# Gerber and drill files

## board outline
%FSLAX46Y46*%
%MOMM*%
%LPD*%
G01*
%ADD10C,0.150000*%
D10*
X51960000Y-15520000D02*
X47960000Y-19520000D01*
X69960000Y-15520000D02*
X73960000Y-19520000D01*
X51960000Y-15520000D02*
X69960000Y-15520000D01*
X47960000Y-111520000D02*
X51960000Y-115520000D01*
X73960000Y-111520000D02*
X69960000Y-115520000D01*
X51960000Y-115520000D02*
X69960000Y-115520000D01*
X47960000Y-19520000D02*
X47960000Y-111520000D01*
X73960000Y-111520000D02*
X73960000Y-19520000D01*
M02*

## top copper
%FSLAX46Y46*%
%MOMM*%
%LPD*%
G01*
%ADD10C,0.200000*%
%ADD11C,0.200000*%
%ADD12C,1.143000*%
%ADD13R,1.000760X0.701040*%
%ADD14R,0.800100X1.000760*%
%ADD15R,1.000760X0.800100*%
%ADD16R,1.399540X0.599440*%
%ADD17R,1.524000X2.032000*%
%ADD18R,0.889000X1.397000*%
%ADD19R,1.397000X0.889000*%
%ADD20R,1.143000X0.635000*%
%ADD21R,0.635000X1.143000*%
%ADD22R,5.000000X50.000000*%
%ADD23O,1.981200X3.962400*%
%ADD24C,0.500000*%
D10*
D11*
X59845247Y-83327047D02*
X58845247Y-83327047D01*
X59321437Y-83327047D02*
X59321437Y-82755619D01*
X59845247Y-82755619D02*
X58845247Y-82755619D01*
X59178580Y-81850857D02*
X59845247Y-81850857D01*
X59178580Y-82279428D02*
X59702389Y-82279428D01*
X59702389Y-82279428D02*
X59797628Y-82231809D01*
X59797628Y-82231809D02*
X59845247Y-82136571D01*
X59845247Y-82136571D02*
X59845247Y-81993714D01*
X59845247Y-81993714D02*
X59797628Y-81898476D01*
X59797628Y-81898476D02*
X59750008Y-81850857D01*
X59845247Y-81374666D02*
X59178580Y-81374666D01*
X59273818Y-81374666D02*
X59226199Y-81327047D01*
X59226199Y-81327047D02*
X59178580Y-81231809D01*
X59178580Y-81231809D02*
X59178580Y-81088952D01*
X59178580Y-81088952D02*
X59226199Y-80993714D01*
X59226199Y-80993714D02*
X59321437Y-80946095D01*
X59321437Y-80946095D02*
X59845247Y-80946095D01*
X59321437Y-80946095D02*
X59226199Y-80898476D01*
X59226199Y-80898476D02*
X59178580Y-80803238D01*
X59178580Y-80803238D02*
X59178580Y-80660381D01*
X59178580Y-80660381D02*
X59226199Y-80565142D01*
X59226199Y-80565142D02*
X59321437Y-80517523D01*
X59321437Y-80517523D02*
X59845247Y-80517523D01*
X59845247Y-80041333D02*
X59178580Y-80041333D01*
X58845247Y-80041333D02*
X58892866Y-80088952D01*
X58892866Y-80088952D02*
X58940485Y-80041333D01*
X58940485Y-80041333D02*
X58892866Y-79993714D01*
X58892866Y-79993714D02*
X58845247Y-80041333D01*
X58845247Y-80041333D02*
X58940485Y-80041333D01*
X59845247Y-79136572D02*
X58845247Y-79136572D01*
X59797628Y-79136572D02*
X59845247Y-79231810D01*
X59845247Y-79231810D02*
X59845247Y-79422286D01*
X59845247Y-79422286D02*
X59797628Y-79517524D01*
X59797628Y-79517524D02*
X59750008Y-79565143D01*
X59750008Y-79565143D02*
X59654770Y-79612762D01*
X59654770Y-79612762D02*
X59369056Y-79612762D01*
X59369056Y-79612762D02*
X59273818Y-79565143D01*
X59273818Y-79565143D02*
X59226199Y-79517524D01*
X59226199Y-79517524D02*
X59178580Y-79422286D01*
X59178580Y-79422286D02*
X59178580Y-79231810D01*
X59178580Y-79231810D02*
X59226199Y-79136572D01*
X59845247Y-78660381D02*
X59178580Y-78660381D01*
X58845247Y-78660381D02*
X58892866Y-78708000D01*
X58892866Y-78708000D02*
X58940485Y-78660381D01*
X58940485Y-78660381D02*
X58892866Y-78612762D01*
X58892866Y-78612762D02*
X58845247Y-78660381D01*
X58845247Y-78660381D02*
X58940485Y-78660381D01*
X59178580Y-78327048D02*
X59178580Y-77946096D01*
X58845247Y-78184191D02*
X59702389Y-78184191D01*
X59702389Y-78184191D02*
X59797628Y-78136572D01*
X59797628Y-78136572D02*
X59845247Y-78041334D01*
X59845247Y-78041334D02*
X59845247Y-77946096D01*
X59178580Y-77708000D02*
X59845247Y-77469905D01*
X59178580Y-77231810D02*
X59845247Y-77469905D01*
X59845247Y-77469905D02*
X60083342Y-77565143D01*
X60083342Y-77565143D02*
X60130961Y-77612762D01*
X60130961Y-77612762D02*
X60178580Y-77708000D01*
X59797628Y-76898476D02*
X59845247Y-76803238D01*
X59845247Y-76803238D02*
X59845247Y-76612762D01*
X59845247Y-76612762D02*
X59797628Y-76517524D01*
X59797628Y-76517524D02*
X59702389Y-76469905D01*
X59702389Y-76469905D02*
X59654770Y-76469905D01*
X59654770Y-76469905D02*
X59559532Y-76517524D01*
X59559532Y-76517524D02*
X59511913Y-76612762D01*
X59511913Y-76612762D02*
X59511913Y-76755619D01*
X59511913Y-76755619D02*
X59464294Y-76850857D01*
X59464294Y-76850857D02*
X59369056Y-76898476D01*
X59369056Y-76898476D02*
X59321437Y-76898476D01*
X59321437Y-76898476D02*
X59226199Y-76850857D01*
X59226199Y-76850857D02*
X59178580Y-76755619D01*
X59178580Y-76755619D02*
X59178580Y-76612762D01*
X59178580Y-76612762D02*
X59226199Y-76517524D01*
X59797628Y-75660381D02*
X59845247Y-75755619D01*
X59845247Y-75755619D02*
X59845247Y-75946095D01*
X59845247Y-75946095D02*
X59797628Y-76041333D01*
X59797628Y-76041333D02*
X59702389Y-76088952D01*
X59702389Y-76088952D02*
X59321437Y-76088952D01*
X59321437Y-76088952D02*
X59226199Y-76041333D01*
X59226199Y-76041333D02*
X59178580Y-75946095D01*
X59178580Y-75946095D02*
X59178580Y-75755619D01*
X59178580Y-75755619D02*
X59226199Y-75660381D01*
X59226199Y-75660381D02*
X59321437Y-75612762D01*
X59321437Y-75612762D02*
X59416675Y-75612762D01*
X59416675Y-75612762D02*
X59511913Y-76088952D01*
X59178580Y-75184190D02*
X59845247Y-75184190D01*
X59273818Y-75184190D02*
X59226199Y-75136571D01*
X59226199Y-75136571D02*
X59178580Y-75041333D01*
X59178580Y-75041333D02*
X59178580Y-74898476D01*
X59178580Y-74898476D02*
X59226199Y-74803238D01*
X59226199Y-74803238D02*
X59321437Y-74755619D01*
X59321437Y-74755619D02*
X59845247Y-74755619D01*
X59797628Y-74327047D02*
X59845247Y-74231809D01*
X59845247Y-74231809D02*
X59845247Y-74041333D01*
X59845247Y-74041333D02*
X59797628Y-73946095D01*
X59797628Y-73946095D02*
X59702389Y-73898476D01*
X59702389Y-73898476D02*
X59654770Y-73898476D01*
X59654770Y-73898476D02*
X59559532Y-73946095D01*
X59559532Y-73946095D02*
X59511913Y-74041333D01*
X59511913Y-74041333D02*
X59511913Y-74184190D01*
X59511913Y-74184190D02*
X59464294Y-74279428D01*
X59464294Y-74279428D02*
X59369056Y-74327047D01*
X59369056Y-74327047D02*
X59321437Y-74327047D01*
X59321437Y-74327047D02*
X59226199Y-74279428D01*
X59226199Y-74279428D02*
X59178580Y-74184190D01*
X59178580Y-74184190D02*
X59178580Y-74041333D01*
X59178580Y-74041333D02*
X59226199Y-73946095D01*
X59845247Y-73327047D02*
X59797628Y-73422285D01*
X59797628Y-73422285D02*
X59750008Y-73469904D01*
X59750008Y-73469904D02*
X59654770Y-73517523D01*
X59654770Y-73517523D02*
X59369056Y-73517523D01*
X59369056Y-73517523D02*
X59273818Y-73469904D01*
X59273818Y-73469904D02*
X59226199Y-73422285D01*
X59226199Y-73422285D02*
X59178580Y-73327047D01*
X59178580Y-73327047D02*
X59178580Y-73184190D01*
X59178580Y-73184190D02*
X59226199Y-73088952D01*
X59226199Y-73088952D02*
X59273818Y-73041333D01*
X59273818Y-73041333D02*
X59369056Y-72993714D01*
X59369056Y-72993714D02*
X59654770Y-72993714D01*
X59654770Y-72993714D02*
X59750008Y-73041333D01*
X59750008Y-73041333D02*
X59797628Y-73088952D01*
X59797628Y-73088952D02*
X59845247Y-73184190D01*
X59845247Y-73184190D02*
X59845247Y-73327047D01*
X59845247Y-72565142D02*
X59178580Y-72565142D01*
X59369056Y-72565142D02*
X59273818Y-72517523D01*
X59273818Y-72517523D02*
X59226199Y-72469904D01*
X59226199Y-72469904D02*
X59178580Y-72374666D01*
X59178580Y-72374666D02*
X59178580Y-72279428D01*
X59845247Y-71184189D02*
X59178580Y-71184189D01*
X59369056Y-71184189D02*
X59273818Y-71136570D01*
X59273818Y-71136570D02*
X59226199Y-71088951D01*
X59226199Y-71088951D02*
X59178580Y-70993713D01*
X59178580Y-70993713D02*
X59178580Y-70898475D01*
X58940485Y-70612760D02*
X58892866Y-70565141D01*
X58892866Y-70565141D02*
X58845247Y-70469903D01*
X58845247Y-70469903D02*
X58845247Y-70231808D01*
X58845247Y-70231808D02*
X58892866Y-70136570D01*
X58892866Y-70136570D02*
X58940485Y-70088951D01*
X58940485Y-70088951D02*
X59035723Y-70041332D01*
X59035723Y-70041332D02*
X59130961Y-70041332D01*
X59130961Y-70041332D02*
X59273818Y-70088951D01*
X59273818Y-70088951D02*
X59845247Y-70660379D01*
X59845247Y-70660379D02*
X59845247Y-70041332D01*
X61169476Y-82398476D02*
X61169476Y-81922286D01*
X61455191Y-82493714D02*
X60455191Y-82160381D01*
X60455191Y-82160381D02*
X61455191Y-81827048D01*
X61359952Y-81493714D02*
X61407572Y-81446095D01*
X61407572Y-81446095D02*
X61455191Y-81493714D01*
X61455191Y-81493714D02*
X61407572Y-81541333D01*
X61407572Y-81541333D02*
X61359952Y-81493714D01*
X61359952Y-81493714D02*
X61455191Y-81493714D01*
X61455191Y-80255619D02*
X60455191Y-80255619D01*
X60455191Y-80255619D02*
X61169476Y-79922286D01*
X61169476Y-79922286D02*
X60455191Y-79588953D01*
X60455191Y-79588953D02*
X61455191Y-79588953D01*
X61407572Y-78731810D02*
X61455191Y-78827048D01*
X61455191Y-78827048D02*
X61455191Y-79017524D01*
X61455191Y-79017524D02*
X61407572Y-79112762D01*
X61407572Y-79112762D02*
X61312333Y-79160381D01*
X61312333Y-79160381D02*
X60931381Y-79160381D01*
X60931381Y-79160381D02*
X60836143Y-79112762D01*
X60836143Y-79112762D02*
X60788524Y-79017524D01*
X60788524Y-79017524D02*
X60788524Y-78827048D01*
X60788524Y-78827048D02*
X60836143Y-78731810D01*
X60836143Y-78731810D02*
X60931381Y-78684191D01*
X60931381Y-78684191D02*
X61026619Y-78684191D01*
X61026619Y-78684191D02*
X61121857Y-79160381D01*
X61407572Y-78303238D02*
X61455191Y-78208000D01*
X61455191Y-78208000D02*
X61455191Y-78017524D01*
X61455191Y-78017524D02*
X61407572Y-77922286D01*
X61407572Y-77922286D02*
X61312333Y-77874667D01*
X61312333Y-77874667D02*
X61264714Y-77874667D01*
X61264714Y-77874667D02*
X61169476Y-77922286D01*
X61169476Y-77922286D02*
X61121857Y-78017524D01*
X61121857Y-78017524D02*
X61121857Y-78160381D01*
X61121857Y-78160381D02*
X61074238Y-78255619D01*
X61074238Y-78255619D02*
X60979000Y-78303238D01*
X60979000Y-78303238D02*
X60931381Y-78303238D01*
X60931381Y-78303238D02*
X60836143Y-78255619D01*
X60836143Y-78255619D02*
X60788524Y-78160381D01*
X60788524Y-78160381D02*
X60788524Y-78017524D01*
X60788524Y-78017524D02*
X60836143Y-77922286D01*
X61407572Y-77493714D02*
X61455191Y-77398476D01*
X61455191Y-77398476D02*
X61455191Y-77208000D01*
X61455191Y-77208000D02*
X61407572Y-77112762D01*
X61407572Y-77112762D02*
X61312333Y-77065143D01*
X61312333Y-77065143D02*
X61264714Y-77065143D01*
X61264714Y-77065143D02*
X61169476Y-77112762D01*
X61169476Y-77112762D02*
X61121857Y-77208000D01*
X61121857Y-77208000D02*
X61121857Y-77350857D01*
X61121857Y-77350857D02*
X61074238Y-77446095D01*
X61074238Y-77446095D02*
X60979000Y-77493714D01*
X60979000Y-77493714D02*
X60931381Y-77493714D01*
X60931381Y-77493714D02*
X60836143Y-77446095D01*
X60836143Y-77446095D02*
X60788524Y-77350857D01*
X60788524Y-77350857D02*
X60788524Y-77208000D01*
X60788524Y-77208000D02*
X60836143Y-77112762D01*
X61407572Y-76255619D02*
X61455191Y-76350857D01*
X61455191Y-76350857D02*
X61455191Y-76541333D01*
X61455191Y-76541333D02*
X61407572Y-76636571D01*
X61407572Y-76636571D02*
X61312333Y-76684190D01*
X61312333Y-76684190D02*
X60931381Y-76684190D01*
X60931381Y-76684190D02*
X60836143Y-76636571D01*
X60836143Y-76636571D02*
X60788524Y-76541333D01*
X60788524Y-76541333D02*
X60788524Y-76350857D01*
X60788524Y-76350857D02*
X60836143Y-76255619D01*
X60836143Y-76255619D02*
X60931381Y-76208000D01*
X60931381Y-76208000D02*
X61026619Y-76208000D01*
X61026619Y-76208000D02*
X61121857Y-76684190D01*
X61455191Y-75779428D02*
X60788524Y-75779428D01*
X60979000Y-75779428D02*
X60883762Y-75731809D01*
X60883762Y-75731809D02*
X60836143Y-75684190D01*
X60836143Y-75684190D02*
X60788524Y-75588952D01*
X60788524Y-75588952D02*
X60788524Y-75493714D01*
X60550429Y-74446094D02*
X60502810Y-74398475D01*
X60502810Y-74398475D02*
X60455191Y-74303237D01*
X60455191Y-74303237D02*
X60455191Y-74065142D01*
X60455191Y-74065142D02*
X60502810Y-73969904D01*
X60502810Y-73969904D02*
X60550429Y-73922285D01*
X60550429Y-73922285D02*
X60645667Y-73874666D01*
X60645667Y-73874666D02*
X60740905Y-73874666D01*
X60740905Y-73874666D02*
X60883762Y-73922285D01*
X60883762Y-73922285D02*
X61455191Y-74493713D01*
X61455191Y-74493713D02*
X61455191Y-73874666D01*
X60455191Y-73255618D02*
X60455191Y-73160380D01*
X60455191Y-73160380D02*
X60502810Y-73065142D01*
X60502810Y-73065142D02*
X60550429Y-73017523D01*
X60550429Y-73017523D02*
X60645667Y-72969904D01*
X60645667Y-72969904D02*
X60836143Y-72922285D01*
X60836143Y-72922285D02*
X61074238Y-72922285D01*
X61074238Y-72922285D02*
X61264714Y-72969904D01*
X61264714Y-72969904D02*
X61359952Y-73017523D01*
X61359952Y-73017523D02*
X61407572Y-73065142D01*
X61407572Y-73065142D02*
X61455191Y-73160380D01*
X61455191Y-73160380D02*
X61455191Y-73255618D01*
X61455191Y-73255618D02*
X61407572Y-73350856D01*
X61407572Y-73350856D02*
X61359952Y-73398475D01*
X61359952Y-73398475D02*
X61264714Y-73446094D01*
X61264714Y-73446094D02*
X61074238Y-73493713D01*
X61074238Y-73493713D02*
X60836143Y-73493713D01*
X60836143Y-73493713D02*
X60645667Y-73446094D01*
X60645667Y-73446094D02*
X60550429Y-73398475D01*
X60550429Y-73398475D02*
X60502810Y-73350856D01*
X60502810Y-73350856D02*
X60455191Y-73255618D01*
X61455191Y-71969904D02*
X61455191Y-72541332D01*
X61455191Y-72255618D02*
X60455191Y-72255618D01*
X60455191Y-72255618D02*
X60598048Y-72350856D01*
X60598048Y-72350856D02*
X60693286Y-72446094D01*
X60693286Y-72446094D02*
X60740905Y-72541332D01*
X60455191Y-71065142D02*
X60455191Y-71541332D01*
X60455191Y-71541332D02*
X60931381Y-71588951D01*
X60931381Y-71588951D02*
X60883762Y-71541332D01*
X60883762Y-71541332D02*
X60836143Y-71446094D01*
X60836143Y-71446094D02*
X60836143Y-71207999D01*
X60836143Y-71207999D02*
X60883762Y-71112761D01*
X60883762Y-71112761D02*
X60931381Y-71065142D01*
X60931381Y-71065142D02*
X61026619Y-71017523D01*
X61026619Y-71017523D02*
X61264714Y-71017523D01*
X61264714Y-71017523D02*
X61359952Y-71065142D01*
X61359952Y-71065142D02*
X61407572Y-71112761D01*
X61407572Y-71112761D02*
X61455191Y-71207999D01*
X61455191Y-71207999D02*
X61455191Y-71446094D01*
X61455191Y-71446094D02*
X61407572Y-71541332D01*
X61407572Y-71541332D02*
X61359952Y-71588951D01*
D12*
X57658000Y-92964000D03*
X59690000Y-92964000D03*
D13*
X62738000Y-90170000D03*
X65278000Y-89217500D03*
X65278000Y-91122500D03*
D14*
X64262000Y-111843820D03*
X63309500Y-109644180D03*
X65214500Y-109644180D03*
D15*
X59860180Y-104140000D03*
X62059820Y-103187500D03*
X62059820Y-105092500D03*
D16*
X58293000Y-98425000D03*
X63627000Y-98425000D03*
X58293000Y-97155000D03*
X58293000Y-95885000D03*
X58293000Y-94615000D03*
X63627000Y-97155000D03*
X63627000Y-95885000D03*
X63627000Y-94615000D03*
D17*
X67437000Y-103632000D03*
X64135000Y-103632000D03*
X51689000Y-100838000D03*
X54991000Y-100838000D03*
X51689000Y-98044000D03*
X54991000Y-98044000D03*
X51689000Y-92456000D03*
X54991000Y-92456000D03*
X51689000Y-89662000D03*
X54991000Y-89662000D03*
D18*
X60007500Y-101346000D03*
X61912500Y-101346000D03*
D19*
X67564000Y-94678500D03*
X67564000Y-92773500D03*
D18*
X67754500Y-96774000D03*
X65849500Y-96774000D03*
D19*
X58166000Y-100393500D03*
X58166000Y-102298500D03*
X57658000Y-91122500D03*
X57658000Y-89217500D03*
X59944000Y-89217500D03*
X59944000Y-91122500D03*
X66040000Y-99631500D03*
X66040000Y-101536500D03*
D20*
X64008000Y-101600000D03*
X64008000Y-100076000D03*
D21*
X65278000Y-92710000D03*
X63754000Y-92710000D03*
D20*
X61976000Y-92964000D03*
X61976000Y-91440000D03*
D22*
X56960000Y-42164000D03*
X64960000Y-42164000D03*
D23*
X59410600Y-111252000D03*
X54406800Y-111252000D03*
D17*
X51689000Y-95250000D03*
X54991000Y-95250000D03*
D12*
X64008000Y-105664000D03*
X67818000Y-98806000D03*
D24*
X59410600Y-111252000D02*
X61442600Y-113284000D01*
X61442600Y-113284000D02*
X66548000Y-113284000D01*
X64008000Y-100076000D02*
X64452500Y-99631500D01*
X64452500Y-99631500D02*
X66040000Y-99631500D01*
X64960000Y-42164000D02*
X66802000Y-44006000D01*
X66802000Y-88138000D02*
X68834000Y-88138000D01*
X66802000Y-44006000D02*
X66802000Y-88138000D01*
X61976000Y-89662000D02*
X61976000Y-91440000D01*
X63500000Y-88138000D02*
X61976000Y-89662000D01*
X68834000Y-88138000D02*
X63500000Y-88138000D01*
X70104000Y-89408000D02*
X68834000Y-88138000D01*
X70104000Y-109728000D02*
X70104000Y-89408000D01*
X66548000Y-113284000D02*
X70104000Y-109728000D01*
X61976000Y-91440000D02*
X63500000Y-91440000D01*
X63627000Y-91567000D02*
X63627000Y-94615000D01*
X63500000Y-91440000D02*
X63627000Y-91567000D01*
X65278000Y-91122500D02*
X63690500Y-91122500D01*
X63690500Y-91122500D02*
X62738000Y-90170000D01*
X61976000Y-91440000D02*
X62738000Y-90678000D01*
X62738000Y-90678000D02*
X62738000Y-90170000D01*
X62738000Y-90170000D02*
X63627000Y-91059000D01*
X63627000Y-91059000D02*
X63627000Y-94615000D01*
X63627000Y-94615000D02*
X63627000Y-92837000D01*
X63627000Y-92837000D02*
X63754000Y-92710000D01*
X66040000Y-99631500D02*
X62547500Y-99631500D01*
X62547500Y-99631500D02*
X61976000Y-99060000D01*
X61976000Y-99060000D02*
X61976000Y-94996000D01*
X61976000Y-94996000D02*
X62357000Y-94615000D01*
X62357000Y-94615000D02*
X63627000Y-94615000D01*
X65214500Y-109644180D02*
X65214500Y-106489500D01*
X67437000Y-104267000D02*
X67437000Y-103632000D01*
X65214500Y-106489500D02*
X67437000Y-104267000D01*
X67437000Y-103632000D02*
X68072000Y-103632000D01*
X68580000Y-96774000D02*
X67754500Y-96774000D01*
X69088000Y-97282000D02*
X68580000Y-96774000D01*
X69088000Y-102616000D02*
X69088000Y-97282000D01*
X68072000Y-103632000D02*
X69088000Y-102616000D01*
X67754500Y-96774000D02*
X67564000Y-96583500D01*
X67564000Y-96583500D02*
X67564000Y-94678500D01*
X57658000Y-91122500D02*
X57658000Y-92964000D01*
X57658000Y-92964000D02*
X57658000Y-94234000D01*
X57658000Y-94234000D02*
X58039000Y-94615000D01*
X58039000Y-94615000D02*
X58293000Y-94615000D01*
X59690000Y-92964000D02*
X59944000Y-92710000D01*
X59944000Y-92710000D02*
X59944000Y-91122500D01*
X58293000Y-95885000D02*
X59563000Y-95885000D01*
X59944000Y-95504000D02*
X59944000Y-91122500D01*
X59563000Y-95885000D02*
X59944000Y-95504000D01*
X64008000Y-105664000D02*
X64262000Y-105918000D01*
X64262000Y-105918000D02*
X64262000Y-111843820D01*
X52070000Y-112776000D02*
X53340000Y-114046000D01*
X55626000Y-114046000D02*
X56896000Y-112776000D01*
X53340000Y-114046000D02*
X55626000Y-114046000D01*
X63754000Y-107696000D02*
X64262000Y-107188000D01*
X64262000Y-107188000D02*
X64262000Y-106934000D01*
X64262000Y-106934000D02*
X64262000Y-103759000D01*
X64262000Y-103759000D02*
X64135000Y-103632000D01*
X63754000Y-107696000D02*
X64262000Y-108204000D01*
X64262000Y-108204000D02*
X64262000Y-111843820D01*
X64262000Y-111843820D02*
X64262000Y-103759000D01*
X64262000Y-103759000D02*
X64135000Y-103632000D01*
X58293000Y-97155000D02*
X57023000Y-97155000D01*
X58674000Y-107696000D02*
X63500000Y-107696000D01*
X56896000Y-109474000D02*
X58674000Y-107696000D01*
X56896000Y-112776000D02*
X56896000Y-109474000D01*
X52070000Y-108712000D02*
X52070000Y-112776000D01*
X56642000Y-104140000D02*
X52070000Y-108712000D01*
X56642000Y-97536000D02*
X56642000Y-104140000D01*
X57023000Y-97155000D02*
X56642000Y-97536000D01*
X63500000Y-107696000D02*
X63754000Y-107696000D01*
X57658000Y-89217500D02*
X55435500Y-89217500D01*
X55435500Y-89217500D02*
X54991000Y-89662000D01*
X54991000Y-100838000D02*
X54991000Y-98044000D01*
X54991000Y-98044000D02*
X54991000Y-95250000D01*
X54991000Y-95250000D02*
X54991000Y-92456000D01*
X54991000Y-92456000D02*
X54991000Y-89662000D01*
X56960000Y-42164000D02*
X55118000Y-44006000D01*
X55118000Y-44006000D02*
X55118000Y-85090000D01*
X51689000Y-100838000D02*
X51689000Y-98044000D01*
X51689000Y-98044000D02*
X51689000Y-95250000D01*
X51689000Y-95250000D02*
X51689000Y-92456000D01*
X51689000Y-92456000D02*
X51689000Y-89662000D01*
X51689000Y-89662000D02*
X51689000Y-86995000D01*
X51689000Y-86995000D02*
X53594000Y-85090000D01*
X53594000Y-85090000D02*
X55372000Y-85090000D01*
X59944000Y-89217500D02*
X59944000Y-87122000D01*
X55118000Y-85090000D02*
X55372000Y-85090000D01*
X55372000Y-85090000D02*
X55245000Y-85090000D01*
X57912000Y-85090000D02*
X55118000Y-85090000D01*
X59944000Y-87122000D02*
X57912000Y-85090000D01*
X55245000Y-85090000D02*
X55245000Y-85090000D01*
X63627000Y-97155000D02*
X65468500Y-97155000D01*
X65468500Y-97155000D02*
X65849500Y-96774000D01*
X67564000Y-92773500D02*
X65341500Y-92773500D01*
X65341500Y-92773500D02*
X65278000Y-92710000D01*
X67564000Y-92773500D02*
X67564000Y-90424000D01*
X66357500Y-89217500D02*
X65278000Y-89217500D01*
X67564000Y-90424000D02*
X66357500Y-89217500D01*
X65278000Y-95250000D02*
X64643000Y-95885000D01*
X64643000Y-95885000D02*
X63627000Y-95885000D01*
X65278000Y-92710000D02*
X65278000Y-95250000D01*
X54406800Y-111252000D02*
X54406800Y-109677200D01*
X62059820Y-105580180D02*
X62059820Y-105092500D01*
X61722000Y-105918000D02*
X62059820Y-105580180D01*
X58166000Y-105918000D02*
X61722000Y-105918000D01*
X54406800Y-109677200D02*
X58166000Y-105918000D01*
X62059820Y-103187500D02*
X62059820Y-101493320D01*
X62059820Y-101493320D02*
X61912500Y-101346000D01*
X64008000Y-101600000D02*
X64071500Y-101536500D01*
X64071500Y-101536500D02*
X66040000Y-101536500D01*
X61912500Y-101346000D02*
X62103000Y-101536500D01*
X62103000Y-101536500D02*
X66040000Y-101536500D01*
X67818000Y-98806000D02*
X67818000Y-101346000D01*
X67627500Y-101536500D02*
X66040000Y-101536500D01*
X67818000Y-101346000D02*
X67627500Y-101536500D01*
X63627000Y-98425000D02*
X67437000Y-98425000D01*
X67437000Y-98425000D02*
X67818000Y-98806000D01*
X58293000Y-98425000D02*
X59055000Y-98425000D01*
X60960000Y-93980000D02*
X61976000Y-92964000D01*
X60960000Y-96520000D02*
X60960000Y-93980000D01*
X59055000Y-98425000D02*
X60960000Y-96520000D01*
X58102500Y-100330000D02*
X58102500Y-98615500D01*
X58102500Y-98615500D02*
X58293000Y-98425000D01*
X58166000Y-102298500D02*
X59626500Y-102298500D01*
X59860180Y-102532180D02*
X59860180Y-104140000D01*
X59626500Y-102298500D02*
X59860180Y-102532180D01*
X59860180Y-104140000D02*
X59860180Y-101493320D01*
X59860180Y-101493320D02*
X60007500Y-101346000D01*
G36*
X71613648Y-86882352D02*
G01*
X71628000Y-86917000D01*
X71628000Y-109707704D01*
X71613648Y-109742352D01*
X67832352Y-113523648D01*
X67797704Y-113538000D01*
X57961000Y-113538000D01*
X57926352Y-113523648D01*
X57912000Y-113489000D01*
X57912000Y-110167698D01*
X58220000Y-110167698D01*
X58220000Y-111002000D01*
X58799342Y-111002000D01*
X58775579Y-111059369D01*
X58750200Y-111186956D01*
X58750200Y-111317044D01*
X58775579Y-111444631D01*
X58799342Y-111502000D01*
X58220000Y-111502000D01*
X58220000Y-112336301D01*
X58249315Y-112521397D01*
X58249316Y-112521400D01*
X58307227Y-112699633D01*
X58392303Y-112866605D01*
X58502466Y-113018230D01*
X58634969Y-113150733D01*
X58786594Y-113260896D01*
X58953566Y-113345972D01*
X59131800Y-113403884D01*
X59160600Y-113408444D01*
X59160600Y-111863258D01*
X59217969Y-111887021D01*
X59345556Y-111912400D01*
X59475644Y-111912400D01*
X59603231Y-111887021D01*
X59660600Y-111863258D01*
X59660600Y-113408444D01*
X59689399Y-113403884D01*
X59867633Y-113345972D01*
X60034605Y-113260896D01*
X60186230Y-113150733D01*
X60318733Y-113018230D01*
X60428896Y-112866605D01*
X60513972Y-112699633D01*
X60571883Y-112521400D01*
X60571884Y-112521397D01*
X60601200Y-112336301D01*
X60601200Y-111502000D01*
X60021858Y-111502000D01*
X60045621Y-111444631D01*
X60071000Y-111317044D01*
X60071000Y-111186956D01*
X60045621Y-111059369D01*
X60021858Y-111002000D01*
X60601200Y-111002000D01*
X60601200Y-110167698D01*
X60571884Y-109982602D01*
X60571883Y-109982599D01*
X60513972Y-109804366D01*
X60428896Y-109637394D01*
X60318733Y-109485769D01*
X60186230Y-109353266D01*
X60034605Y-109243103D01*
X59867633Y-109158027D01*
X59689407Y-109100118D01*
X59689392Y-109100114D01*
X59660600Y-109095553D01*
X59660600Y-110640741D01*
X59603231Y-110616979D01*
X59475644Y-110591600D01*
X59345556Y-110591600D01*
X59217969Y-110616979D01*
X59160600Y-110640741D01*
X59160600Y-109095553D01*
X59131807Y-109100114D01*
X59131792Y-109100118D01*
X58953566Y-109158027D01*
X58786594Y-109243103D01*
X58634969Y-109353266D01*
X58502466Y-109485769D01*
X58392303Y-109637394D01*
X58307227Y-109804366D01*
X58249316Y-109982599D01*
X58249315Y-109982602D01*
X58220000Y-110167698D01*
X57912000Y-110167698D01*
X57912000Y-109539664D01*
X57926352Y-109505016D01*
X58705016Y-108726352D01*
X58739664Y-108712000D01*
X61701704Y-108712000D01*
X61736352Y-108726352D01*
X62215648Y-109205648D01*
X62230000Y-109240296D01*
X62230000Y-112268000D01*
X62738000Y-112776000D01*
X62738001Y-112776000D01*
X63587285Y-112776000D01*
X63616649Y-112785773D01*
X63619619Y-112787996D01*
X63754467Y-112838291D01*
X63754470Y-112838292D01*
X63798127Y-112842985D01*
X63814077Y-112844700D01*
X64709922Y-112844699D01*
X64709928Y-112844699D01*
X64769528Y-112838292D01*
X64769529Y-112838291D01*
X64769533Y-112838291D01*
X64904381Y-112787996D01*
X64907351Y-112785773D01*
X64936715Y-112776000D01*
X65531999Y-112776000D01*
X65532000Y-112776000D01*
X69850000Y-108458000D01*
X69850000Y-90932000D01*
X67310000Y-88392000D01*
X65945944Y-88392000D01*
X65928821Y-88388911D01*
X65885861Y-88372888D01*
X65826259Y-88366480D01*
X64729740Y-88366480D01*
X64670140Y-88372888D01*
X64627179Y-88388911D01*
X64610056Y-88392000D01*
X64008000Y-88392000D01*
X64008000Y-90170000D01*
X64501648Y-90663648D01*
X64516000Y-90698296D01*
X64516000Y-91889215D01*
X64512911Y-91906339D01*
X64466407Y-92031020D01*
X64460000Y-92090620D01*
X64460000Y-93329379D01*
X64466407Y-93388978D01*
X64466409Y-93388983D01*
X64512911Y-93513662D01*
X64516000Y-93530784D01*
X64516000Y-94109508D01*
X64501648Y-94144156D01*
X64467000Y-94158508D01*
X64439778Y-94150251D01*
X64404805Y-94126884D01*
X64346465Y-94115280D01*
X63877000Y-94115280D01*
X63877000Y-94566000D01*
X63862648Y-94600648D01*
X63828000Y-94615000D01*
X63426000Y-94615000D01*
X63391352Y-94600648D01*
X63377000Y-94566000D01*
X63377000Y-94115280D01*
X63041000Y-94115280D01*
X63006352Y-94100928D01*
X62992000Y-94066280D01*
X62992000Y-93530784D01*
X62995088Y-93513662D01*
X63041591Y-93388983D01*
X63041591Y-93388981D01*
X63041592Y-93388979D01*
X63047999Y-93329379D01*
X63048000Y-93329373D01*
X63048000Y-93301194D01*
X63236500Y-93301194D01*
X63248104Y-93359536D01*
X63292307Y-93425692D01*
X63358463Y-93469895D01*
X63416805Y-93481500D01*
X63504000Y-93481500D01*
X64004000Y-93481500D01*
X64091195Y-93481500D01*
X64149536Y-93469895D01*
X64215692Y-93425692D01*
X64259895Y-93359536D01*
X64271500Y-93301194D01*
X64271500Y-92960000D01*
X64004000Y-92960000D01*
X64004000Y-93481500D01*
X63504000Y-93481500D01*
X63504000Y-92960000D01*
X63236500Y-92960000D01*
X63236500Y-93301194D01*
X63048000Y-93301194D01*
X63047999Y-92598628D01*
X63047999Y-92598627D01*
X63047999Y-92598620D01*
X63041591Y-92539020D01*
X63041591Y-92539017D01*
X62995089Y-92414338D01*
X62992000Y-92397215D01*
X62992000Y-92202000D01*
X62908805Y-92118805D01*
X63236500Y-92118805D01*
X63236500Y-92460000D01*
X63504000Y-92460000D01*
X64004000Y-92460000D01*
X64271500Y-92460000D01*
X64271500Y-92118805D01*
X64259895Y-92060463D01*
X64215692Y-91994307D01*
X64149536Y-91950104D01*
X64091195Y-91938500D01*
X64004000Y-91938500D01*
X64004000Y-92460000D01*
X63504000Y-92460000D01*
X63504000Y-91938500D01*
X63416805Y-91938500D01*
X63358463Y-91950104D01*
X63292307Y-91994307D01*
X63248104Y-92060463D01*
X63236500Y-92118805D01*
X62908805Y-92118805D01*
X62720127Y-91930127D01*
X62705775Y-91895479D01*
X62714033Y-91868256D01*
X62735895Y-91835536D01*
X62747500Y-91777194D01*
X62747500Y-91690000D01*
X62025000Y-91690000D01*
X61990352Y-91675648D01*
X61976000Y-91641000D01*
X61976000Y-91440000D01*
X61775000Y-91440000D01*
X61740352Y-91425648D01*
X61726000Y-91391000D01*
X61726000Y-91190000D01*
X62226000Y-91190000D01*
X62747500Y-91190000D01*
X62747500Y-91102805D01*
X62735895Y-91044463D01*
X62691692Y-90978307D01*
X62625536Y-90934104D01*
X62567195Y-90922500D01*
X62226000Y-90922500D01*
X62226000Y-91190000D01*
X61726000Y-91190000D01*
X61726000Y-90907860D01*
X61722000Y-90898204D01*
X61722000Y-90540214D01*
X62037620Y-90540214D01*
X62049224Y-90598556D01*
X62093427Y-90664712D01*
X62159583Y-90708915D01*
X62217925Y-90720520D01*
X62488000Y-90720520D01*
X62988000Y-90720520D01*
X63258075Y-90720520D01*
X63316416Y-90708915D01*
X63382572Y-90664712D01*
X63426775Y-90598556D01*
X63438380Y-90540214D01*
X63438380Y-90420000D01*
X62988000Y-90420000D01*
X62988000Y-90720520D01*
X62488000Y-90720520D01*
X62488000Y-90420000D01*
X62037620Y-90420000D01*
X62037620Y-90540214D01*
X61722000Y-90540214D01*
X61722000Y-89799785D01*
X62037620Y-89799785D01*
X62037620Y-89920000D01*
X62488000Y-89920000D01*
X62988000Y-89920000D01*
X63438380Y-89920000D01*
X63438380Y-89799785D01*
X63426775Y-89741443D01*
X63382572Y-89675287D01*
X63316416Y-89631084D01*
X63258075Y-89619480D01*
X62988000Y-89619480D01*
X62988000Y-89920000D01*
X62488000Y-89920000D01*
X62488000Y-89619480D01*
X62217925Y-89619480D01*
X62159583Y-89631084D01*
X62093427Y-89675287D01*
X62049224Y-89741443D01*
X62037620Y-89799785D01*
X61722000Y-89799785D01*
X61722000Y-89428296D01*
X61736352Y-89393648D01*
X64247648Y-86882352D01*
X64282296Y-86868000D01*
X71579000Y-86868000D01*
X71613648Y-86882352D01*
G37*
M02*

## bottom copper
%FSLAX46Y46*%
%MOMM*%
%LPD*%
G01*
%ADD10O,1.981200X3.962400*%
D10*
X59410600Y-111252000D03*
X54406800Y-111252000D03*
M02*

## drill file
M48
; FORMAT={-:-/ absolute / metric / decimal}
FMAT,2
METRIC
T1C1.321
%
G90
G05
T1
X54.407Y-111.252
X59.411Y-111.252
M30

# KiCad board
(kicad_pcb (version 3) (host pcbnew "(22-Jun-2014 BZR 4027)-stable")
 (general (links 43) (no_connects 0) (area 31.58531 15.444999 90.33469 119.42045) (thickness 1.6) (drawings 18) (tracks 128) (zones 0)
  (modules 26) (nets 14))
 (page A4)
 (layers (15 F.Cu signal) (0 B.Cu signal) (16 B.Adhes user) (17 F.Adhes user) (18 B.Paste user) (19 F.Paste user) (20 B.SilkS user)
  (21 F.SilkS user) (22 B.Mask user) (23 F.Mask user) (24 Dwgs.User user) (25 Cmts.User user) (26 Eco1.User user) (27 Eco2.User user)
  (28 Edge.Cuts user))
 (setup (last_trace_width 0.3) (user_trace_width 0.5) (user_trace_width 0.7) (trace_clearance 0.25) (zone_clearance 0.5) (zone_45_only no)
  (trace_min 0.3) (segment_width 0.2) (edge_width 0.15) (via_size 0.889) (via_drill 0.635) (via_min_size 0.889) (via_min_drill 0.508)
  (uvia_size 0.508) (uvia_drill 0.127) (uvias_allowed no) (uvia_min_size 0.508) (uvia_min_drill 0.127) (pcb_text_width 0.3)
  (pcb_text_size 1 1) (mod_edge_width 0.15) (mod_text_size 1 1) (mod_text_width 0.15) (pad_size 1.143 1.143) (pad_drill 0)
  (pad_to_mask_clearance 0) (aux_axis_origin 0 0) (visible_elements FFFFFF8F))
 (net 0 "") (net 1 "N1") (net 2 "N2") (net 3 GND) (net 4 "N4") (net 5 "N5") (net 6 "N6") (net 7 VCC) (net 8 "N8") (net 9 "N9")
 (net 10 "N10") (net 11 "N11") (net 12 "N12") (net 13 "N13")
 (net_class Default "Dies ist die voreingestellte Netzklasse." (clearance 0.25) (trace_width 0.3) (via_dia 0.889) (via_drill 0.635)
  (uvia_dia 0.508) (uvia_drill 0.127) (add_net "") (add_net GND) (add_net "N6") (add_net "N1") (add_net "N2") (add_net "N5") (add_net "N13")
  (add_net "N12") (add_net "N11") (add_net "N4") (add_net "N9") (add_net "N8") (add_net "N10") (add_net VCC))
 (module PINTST (layer F.Cu) (at 57.658 92.964)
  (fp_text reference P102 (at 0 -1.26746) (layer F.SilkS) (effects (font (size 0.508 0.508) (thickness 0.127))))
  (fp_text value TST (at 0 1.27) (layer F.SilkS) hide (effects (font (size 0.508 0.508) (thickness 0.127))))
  (pad 1 smd circle (at 0 0) (size 1.143 1.143) (layers F.Cu F.Paste F.Mask) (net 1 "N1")))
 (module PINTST (layer F.Cu) (at 59.69 92.964)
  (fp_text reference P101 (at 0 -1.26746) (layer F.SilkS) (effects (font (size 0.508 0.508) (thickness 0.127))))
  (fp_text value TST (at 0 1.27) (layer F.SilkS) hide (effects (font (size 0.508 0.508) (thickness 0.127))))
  (pad 1 smd circle (at 0 0) (size 1.143 1.143) (layers F.Cu F.Paste F.Mask) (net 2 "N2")))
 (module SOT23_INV (layer F.Cu) (at 64.008 90.17 90)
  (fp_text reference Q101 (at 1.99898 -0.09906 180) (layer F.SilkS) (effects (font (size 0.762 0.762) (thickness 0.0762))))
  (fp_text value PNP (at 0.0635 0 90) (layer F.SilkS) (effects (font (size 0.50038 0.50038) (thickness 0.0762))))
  (pad 3 smd rect (at 0 -1.27 90) (size 0.70104 1.00076) (layers F.Cu F.Paste F.Mask) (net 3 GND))
  (pad 1 smd rect (at 0.9525 1.27 90) (size 0.70104 1.00076) (layers F.Cu F.Paste F.Mask) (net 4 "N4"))
  (pad 2 smd rect (at -0.9525 1.27 90) (size 0.70104 1.00076) (layers F.Cu F.Paste F.Mask) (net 3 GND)))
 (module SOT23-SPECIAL (layer F.Cu) (at 64.262 110.744 180)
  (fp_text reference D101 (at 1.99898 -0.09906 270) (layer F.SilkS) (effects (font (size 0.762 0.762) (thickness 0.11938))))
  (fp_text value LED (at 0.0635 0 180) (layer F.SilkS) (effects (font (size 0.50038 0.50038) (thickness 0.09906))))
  (pad 2 smd rect (at 0 -1.09982 180) (size 0.8001 1.00076) (layers F.Cu F.Paste F.Mask) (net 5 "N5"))
  (pad 3 smd rect (at 0.9525 1.09982 180) (size 0.8001 1.00076) (layers F.Cu F.Paste F.Mask))
  (pad 1 smd rect (at -0.9525 1.09982 180) (size 0.8001 1.00076) (layers F.Cu F.Paste F.Mask) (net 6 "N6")))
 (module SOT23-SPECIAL (layer F.Cu) (at 60.96 104.14 90)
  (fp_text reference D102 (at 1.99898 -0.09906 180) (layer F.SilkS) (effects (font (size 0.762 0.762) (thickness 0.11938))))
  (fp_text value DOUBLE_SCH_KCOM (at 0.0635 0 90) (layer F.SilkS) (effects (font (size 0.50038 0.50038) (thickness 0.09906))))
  (pad 2 smd rect (at 0 -1.09982 90) (size 0.8001 1.00076) (layers F.Cu F.Paste F.Mask) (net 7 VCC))
  (pad 3 smd rect (at 0.9525 1.09982 90) (size 0.8001 1.00076) (layers F.Cu F.Paste F.Mask) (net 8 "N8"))
  (pad 1 smd rect (at -0.9525 1.09982 90) (size 0.8001 1.00076) (layers F.Cu F.Paste F.Mask) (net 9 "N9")))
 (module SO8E (layer F.Cu) (at 60.96 96.52 90)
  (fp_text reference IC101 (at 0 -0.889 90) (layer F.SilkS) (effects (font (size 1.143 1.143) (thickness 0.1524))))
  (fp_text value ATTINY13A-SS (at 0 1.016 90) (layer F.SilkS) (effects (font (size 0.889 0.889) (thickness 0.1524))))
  (pad 8 smd rect (at -1.905 -2.667 90) (size 0.59944 1.39954) (layers F.Cu F.Paste F.Mask) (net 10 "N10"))
  (pad 1 smd rect (at -1.905 2.667 90) (size 0.59944 1.39954) (layers F.Cu F.Paste F.Mask) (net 8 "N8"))
  (pad 7 smd rect (at -0.635 -2.667 90) (size 0.59944 1.39954) (layers F.Cu F.Paste F.Mask) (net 5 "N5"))
  (pad 6 smd rect (at 0.635 -2.667 90) (size 0.59944 1.39954) (layers F.Cu F.Paste F.Mask) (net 2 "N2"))
  (pad 5 smd rect (at 1.905 -2.667 90) (size 0.59944 1.39954) (layers F.Cu F.Paste F.Mask) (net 1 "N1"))
  (pad 2 smd rect (at -0.635 2.667 90) (size 0.59944 1.39954) (layers F.Cu F.Paste F.Mask) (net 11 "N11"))
  (pad 3 smd rect (at 0.635 2.667 90) (size 0.59944 1.39954) (layers F.Cu F.Paste F.Mask) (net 4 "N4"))
  (pad 4 smd rect (at 1.905 2.667 90) (size 0.59944 1.39954) (layers F.Cu F.Paste F.Mask) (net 3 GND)))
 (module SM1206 (layer F.Cu) (at 65.786 103.632 180)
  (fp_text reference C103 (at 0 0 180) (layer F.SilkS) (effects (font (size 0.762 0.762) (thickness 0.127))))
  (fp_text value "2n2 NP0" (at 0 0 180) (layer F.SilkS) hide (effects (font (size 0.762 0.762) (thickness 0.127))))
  (pad 1 smd rect (at -1.651 0 180) (size 1.524 2.032) (layers F.Cu F.Paste F.Mask) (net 6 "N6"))
  (pad 2 smd rect (at 1.651 0 180) (size 1.524 2.032) (layers F.Cu F.Paste F.Mask) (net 5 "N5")))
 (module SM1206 (layer F.Cu) (at 53.34 100.838)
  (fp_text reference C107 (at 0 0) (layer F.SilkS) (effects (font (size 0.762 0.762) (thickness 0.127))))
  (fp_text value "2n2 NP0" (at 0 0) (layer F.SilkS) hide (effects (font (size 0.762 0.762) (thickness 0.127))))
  (pad 1 smd rect (at -1.651 0) (size 1.524 2.032) (layers F.Cu F.Paste F.Mask) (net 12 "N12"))
  (pad 2 smd rect (at 1.651 0) (size 1.524 2.032) (layers F.Cu F.Paste F.Mask) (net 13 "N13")))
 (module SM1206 (layer F.Cu) (at 53.34 98.044)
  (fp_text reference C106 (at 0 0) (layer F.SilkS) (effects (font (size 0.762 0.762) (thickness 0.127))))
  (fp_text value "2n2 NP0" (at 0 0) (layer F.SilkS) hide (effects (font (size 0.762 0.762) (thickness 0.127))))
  (pad 1 smd rect (at -1.651 0) (size 1.524 2.032) (layers F.Cu F.Paste F.Mask) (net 12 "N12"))
  (pad 2 smd rect (at 1.651 0) (size 1.524 2.032) (layers F.Cu F.Paste F.Mask) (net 13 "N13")))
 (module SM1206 (layer F.Cu) (at 53.34 92.456)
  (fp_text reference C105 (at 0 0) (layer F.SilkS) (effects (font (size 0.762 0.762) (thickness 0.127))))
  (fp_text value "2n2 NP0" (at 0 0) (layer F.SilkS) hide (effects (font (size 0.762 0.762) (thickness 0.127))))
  (pad 1 smd rect (at -1.651 0) (size 1.524 2.032) (layers F.Cu F.Paste F.Mask) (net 12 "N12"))
  (pad 2 smd rect (at 1.651 0) (size 1.524 2.032) (layers F.Cu F.Paste F.Mask) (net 13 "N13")))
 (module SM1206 (layer F.Cu) (at 53.34 89.662)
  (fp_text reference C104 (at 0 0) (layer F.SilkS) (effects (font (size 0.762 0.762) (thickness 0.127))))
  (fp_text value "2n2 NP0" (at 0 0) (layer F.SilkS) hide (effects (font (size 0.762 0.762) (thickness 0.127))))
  (pad 1 smd rect (at -1.651 0) (size 1.524 2.032) (layers F.Cu F.Paste F.Mask) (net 12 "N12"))
  (pad 2 smd rect (at 1.651 0) (size 1.524 2.032) (layers F.Cu F.Paste F.Mask) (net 13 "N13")))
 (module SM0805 (layer F.Cu) (at 60.96 101.346)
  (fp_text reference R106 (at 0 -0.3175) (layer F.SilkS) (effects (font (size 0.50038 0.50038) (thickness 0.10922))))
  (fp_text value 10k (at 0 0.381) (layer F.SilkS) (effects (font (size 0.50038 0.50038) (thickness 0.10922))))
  (pad 1 smd rect (at -0.9525 0) (size 0.889 1.397) (layers F.Cu F.Paste F.Mask) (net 7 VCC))
  (pad 2 smd rect (at 0.9525 0) (size 0.889 1.397) (layers F.Cu F.Paste F.Mask) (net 8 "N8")))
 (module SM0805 (layer F.Cu) (at 67.564 93.726 90)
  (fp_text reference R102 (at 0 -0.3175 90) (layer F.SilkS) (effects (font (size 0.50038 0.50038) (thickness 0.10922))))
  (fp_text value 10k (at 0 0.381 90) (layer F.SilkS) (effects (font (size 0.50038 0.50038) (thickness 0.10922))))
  (pad 1 smd rect (at -0.9525 0 90) (size 0.889 1.397) (layers F.Cu F.Paste F.Mask) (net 6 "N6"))
  (pad 2 smd rect (at 0.9525 0 90) (size 0.889 1.397) (layers F.Cu F.Paste F.Mask) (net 4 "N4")))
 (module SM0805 (layer F.Cu) (at 66.802 96.774 180)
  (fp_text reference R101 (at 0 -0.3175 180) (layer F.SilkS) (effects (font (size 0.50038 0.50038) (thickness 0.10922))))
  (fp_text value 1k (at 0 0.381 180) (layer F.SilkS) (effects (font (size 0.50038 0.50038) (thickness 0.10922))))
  (pad 1 smd rect (at -0.9525 0 180) (size 0.889 1.397) (layers F.Cu F.Paste F.Mask) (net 6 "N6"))
  (pad 2 smd rect (at 0.9525 0 180) (size 0.889 1.397) (layers F.Cu F.Paste F.Mask) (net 11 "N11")))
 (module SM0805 (layer F.Cu) (at 58.166 101.346 270)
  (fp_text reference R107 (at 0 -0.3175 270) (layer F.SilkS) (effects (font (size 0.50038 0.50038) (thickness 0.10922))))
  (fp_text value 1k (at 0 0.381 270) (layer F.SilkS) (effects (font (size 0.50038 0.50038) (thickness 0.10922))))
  (pad 1 smd rect (at -0.9525 0 270) (size 0.889 1.397) (layers F.Cu F.Paste F.Mask) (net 10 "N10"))
  (pad 2 smd rect (at 0.9525 0 270) (size 0.889 1.397) (layers F.Cu F.Paste F.Mask) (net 7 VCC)))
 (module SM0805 (layer F.Cu) (at 57.658 90.17 90)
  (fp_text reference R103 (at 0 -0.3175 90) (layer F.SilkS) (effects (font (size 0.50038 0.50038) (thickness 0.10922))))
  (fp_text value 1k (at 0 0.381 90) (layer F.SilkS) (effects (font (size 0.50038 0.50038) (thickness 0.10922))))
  (pad 1 smd rect (at -0.9525 0 90) (size 0.889 1.397) (layers F.Cu F.Paste F.Mask) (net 1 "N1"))
  (pad 2 smd rect (at 0.9525 0 90) (size 0.889 1.397) (layers F.Cu F.Paste F.Mask) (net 13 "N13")))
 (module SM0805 (layer F.Cu) (at 59.944 90.17 270)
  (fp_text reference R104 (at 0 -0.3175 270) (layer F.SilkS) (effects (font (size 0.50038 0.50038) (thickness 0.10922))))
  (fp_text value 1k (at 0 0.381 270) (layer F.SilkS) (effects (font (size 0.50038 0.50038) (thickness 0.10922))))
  (pad 1 smd rect (at -0.9525 0 270) (size 0.889 1.397) (layers F.Cu F.Paste F.Mask) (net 12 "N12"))
  (pad 2 smd rect (at 0.9525 0 270) (size 0.889 1.397) (layers F.Cu F.Paste F.Mask) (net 2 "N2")))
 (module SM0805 (layer F.Cu) (at 66.04 100.584 270)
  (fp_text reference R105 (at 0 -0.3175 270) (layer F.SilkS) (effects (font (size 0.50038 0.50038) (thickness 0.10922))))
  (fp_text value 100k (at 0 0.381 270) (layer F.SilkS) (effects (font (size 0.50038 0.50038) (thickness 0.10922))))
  (pad 1 smd rect (at -0.9525 0 270) (size 0.889 1.397) (layers F.Cu F.Paste F.Mask) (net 3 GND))
  (pad 2 smd rect (at 0.9525 0 270) (size 0.889 1.397) (layers F.Cu F.Paste F.Mask) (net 8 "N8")))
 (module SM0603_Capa (layer F.Cu) (at 64.008 100.838 90)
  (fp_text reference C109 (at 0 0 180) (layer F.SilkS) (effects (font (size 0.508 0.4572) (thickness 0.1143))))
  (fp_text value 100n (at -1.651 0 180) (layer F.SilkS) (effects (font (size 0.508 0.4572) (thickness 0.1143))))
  (pad 1 smd rect (at -0.762 0 90) (size 0.635 1.143) (layers F.Cu F.Paste F.Mask) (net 8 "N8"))
  (pad 2 smd rect (at 0.762 0 90) (size 0.635 1.143) (layers F.Cu F.Paste F.Mask) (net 3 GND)))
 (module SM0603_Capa (layer F.Cu) (at 64.516 92.71 180)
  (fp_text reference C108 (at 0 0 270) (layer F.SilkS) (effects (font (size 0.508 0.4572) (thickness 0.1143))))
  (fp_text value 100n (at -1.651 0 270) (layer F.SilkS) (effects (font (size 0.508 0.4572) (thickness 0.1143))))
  (pad 1 smd rect (at -0.762 0 180) (size 0.635 1.143) (layers F.Cu F.Paste F.Mask) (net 4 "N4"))
  (pad 2 smd rect (at 0.762 0 180) (size 0.635 1.143) (layers F.Cu F.Paste F.Mask) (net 3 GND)))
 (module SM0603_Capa (layer F.Cu) (at 61.976 92.202 90)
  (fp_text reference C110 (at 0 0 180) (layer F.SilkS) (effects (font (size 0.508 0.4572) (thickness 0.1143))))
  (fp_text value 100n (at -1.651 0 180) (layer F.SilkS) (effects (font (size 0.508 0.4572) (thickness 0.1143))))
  (pad 1 smd rect (at -0.762 0 90) (size 0.635 1.143) (layers F.Cu F.Paste F.Mask) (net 10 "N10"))
  (pad 2 smd rect (at 0.762 0 90) (size 0.635 1.143) (layers F.Cu F.Paste F.Mask) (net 3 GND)))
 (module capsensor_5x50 (layer F.Cu) (at 60.96 42.164)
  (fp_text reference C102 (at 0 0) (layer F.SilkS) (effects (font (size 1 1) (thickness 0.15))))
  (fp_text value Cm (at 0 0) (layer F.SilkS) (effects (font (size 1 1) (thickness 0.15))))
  (pad 1 smd rect (at -4 0) (size 5 50) (layers F.Cu F.Paste F.Mask) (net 12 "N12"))
  (pad 2 smd rect (at 4 0) (size 5 50) (layers F.Cu F.Paste F.Mask) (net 3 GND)))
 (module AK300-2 (layer F.Cu) (at 56.896 111.252 180)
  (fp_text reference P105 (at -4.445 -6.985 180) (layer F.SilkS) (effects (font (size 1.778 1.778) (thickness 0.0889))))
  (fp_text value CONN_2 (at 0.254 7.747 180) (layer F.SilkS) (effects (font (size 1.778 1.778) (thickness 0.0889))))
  (pad 1 thru_hole oval (at -2.5146 0 180) (size 1.9812 3.9624) (drill 1.3208) (layers *.Cu F.Paste F.SilkS F.Mask) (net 3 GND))
  (pad 2 thru_hole oval (at 2.4892 0 180) (size 1.9812 3.9624) (drill 1.3208) (layers *.Cu F.Paste F.SilkS F.Mask) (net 9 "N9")))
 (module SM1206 (layer F.Cu) (at 53.34 95.25)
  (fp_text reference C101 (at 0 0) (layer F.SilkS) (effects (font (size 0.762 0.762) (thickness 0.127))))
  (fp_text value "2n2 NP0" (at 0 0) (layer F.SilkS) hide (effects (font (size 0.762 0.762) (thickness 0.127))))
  (pad 1 smd rect (at -1.651 0) (size 1.524 2.032) (layers F.Cu F.Paste F.Mask) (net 12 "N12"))
  (pad 2 smd rect (at 1.651 0) (size 1.524 2.032) (layers F.Cu F.Paste F.Mask) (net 13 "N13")))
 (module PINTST (layer F.Cu) (at 64.008 105.664)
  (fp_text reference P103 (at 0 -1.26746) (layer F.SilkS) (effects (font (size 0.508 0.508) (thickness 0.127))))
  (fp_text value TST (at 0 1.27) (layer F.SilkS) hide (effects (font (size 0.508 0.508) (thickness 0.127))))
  (pad 1 smd circle (at 0 0) (size 1.143 1.143) (layers F.Cu F.Paste F.Mask) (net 5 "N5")))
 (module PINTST (layer F.Cu) (at 67.818 98.806)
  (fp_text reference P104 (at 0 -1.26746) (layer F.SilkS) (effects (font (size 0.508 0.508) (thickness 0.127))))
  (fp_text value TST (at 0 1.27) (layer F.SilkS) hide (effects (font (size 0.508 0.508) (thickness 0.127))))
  (pad 1 smd circle (at 0 0) (size 1.143 1.143) (layers F.Cu F.Paste F.Mask) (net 8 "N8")))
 (gr_line (start 51.96 15.52) (end 47.96 19.52) (angle 90) (layer Edge.Cuts) (width 0.15))
 (gr_line (start 69.96 15.52) (end 73.96 19.52) (angle 90) (layer Edge.Cuts) (width 0.15))
 (gr_line (start 51.96 15.52) (end 69.96 15.52) (angle 90) (layer Edge.Cuts) (width 0.15))
 (gr_line (start 47.96 111.52) (end 51.96 115.52) (angle 90) (layer Edge.Cuts) (width 0.15))
 (gr_line (start 73.96 111.52) (end 69.96 115.52) (angle 90) (layer Edge.Cuts) (width 0.15))
 (gr_line (start 51.96 115.52) (end 69.96 115.52) (angle 90) (layer Edge.Cuts) (width 0.15))
 (gr_line (start 47.96 19.52) (end 47.96 111.52) (angle 90) (layer Edge.Cuts) (width 0.15))
 (gr_line (start 73.96 111.52) (end 73.96 19.52) (angle 90) (layer Edge.Cuts) (width 0.15))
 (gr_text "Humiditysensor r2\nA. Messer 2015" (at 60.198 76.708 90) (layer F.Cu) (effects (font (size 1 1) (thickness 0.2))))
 (segment (start 59.4106 111.252) (end 61.4426 113.284) (width 0.5) (layer F.Cu) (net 3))
 (segment (start 61.4426 113.284) (end 66.548 113.284) (width 0.5) (layer F.Cu) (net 3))
 (segment (start 64.008 100.076) (end 64.4525 99.6315) (width 0.5) (layer F.Cu) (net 3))
 (segment (start 64.4525 99.6315) (end 66.04 99.6315) (width 0.5) (layer F.Cu) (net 3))
 (segment (start 64.96 42.164) (end 66.802 44.006) (width 0.5) (layer F.Cu) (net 3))
 (segment (start 66.802 88.138) (end 68.834 88.138) (width 0.5) (layer F.Cu) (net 3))
 (segment (start 66.802 44.006) (end 66.802 88.138) (width 0.5) (layer F.Cu) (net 3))
 (segment (start 61.976 89.662) (end 61.976 91.44) (width 0.5) (layer F.Cu) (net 3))
 (segment (start 63.5 88.138) (end 61.976 89.662) (width 0.5) (layer F.Cu) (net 3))
 (segment (start 68.834 88.138) (end 63.5 88.138) (width 0.5) (layer F.Cu) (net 3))
 (segment (start 70.104 89.408) (end 68.834 88.138) (width 0.5) (layer F.Cu) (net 3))
 (segment (start 70.104 109.728) (end 70.104 89.408) (width 0.5) (layer F.Cu) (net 3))
 (segment (start 66.548 113.284) (end 70.104 109.728) (width 0.5) (layer F.Cu) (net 3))
 (segment (start 61.976 91.44) (end 63.5 91.44) (width 0.5) (layer F.Cu) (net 3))
 (segment (start 63.627 91.567) (end 63.627 94.615) (width 0.5) (layer F.Cu) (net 3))
 (segment (start 63.5 91.44) (end 63.627 91.567) (width 0.5) (layer F.Cu) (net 3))
 (segment (start 65.278 91.1225) (end 63.6905 91.1225) (width 0.5) (layer F.Cu) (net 3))
 (segment (start 63.6905 91.1225) (end 62.738 90.17) (width 0.5) (layer F.Cu) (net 3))
 (segment (start 61.976 91.44) (end 62.738 90.678) (width 0.5) (layer F.Cu) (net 3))
 (segment (start 62.738 90.678) (end 62.738 90.17) (width 0.5) (layer F.Cu) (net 3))
 (segment (start 62.738 90.17) (end 63.627 91.059) (width 0.5) (layer F.Cu) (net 3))
 (segment (start 63.627 91.059) (end 63.627 94.615) (width 0.5) (layer F.Cu) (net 3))
 (segment (start 63.627 94.615) (end 63.627 92.837) (width 0.5) (layer F.Cu) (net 3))
 (segment (start 63.627 92.837) (end 63.754 92.71) (width 0.5) (layer F.Cu) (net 3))
 (segment (start 66.04 99.6315) (end 62.5475 99.6315) (width 0.5) (layer F.Cu) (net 3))
 (segment (start 62.5475 99.6315) (end 61.976 99.06) (width 0.5) (layer F.Cu) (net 3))
 (segment (start 61.976 99.06) (end 61.976 94.996) (width 0.5) (layer F.Cu) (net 3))
 (segment (start 61.976 94.996) (end 62.357 94.615) (width 0.5) (layer F.Cu) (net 3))
 (segment (start 62.357 94.615) (end 63.627 94.615) (width 0.5) (layer F.Cu) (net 3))
 (segment (start 65.2145 109.64418) (end 65.2145 106.4895) (width 0.5) (layer F.Cu) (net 6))
 (segment (start 67.437 104.267) (end 67.437 103.632) (width 0.5) (layer F.Cu) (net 6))
 (segment (start 65.2145 106.4895) (end 67.437 104.267) (width 0.5) (layer F.Cu) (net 6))
 (segment (start 67.437 103.632) (end 68.072 103.632) (width 0.5) (layer F.Cu) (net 6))
 (segment (start 68.58 96.774) (end 67.7545 96.774) (width 0.5) (layer F.Cu) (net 6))
 (segment (start 69.088 97.282) (end 68.58 96.774) (width 0.5) (layer F.Cu) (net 6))
 (segment (start 69.088 102.616) (end 69.088 97.282) (width 0.5) (layer F.Cu) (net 6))
 (segment (start 68.072 103.632) (end 69.088 102.616) (width 0.5) (layer F.Cu) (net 6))
 (segment (start 67.7545 96.774) (end 67.564 96.5835) (width 0.5) (layer F.Cu) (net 6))
 (segment (start 67.564 96.5835) (end 67.564 94.6785) (width 0.5) (layer F.Cu) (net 6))
 (segment (start 57.658 91.1225) (end 57.658 92.964) (width 0.5) (layer F.Cu) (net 1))
 (segment (start 57.658 92.964) (end 57.658 94.234) (width 0.5) (layer F.Cu) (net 1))
 (segment (start 57.658 94.234) (end 58.039 94.615) (width 0.5) (layer F.Cu) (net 1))
 (segment (start 58.039 94.615) (end 58.293 94.615) (width 0.5) (layer F.Cu) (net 1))
 (segment (start 59.69 92.964) (end 59.944 92.71) (width 0.5) (layer F.Cu) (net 2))
 (segment (start 59.944 92.71) (end 59.944 91.1225) (width 0.5) (layer F.Cu) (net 2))
 (segment (start 58.293 95.885) (end 59.563 95.885) (width 0.5) (layer F.Cu) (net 2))
 (segment (start 59.944 95.504) (end 59.944 91.1225) (width 0.5) (layer F.Cu) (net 2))
 (segment (start 59.563 95.885) (end 59.944 95.504) (width 0.5) (layer F.Cu) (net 2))
 (segment (start 64.008 105.664) (end 64.262 105.918) (width 0.5) (layer F.Cu) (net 5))
 (segment (start 64.262 105.918) (end 64.262 111.84382) (width 0.5) (layer F.Cu) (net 5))
 (segment (start 52.07 112.776) (end 53.34 114.046) (width 0.5) (layer F.Cu) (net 5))
 (segment (start 55.626 114.046) (end 56.896 112.776) (width 0.5) (layer F.Cu) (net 5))
 (segment (start 53.34 114.046) (end 55.626 114.046) (width 0.5) (layer F.Cu) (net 5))
 (segment (start 63.754 107.696) (end 64.262 107.188) (width 0.5) (layer F.Cu) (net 5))
 (segment (start 64.262 107.188) (end 64.262 106.934) (width 0.5) (layer F.Cu) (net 5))
 (segment (start 64.262 106.934) (end 64.262 103.759) (width 0.5) (layer F.Cu) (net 5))
 (segment (start 64.262 103.759) (end 64.135 103.632) (width 0.5) (layer F.Cu) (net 5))
 (segment (start 63.754 107.696) (end 64.262 108.204) (width 0.5) (layer F.Cu) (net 5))
 (segment (start 64.262 108.204) (end 64.262 111.84382) (width 0.5) (layer F.Cu) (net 5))
 (segment (start 64.262 111.84382) (end 64.262 103.759) (width 0.5) (layer F.Cu) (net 5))
 (segment (start 64.262 103.759) (end 64.135 103.632) (width 0.5) (layer F.Cu) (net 5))
 (segment (start 58.293 97.155) (end 57.023 97.155) (width 0.5) (layer F.Cu) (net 5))
 (segment (start 58.674 107.696) (end 63.5 107.696) (width 0.5) (layer F.Cu) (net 5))
 (segment (start 56.896 109.474) (end 58.674 107.696) (width 0.5) (layer F.Cu) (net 5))
 (segment (start 56.896 112.776) (end 56.896 109.474) (width 0.5) (layer F.Cu) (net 5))
 (segment (start 52.07 108.712) (end 52.07 112.776) (width 0.5) (layer F.Cu) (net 5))
 (segment (start 56.642 104.14) (end 52.07 108.712) (width 0.5) (layer F.Cu) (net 5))
 (segment (start 56.642 97.536) (end 56.642 104.14) (width 0.5) (layer F.Cu) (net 5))
 (segment (start 57.023 97.155) (end 56.642 97.536) (width 0.5) (layer F.Cu) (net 5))
 (segment (start 63.5 107.696) (end 63.754 107.696) (width 0.5) (layer F.Cu) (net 5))
 (segment (start 57.658 89.2175) (end 55.4355 89.2175) (width 0.5) (layer F.Cu) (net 13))
 (segment (start 55.4355 89.2175) (end 54.991 89.662) (width 0.5) (layer F.Cu) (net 13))
 (segment (start 54.991 100.838) (end 54.991 98.044) (width 0.5) (layer F.Cu) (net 13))
 (segment (start 54.991 98.044) (end 54.991 95.25) (width 0.5) (layer F.Cu) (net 13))
 (segment (start 54.991 95.25) (end 54.991 92.456) (width 0.5) (layer F.Cu) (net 13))
 (segment (start 54.991 92.456) (end 54.991 89.662) (width 0.5) (layer F.Cu) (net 13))
 (segment (start 56.96 42.164) (end 55.118 44.006) (width 0.5) (layer F.Cu) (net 12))
 (segment (start 55.118 44.006) (end 55.118 85.09) (width 0.5) (layer F.Cu) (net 12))
 (segment (start 51.689 100.838) (end 51.689 98.044) (width 0.5) (layer F.Cu) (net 12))
 (segment (start 51.689 98.044) (end 51.689 95.25) (width 0.5) (layer F.Cu) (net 12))
 (segment (start 51.689 95.25) (end 51.689 92.456) (width 0.5) (layer F.Cu) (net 12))
 (segment (start 51.689 92.456) (end 51.689 89.662) (width 0.5) (layer F.Cu) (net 12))
 (segment (start 51.689 89.662) (end 51.689 86.995) (width 0.5) (layer F.Cu) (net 12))
 (segment (start 51.689 86.995) (end 53.594 85.09) (width 0.5) (layer F.Cu) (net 12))
 (segment (start 53.594 85.09) (end 55.372 85.09) (width 0.5) (layer F.Cu) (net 12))
 (segment (start 59.944 89.2175) (end 59.944 87.122) (width 0.5) (layer F.Cu) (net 12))
 (segment (start 55.118 85.09) (end 55.372 85.09) (width 0.5) (layer F.Cu) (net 12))
 (segment (start 55.372 85.09) (end 55.245 85.09) (width 0.5) (layer F.Cu) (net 12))
 (segment (start 57.912 85.09) (end 55.118 85.09) (width 0.5) (layer F.Cu) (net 12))
 (segment (start 59.944 87.122) (end 57.912 85.09) (width 0.5) (layer F.Cu) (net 12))
 (segment (start 55.245 85.09) (end 55.245 85.09) (width 0.5) (layer F.Cu) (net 12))
 (segment (start 63.627 97.155) (end 65.4685 97.155) (width 0.5) (layer F.Cu) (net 11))
 (segment (start 65.4685 97.155) (end 65.8495 96.774) (width 0.5) (layer F.Cu) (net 11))
 (segment (start 67.564 92.7735) (end 65.3415 92.7735) (width 0.5) (layer F.Cu) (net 4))
 (segment (start 65.3415 92.7735) (end 65.278 92.71) (width 0.5) (layer F.Cu) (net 4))
 (segment (start 67.564 92.7735) (end 67.564 90.424) (width 0.5) (layer F.Cu) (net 4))
 (segment (start 66.3575 89.2175) (end 65.278 89.2175) (width 0.5) (layer F.Cu) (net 4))
 (segment (start 67.564 90.424) (end 66.3575 89.2175) (width 0.5) (layer F.Cu) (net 4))
 (segment (start 65.278 95.25) (end 64.643 95.885) (width 0.5) (layer F.Cu) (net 4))
 (segment (start 64.643 95.885) (end 63.627 95.885) (width 0.5) (layer F.Cu) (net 4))
 (segment (start 65.278 92.71) (end 65.278 95.25) (width 0.5) (layer F.Cu) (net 4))
 (segment (start 54.4068 111.252) (end 54.4068 109.6772) (width 0.5) (layer F.Cu) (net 9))
 (segment (start 62.05982 105.58018) (end 62.05982 105.0925) (width 0.5) (layer F.Cu) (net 9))
 (segment (start 61.722 105.918) (end 62.05982 105.58018) (width 0.5) (layer F.Cu) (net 9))
 (segment (start 58.166 105.918) (end 61.722 105.918) (width 0.5) (layer F.Cu) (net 9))
 (segment (start 54.4068 109.6772) (end 58.166 105.918) (width 0.5) (layer F.Cu) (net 9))
 (segment (start 62.05982 103.1875) (end 62.05982 101.49332) (width 0.5) (layer F.Cu) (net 8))
 (segment (start 62.05982 101.49332) (end 61.9125 101.346) (width 0.5) (layer F.Cu) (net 8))
 (segment (start 64.008 101.6) (end 64.0715 101.5365) (width 0.5) (layer F.Cu) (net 8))
 (segment (start 64.0715 101.5365) (end 66.04 101.5365) (width 0.5) (layer F.Cu) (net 8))
 (segment (start 61.9125 101.346) (end 62.103 101.5365) (width 0.5) (layer F.Cu) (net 8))
 (segment (start 62.103 101.5365) (end 66.04 101.5365) (width 0.5) (layer F.Cu) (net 8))
 (segment (start 67.818 98.806) (end 67.818 101.346) (width 0.5) (layer F.Cu) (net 8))
 (segment (start 67.6275 101.5365) (end 66.04 101.5365) (width 0.5) (layer F.Cu) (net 8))
 (segment (start 67.818 101.346) (end 67.6275 101.5365) (width 0.5) (layer F.Cu) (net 8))
 (segment (start 63.627 98.425) (end 67.437 98.425) (width 0.5) (layer F.Cu) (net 8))
 (segment (start 67.437 98.425) (end 67.818 98.806) (width 0.5) (layer F.Cu) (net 8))
 (segment (start 58.293 98.425) (end 59.055 98.425) (width 0.5) (layer F.Cu) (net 10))
 (segment (start 60.96 93.98) (end 61.976 92.964) (width 0.5) (layer F.Cu) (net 10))
 (segment (start 60.96 96.52) (end 60.96 93.98) (width 0.5) (layer F.Cu) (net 10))
 (segment (start 59.055 98.425) (end 60.96 96.52) (width 0.5) (layer F.Cu) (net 10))
 (segment (start 58.1025 100.33) (end 58.1025 98.6155) (width 0.5) (layer F.Cu) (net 10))
 (segment (start 58.1025 98.6155) (end 58.293 98.425) (width 0.5) (layer F.Cu) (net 10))
 (segment (start 58.166 102.2985) (end 59.6265 102.2985) (width 0.5) (layer F.Cu) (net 7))
 (segment (start 59.86018 102.53218) (end 59.86018 104.14) (width 0.5) (layer F.Cu) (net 7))
 (segment (start 59.6265 102.2985) (end 59.86018 102.53218) (width 0.5) (layer F.Cu) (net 7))
 (segment (start 59.86018 104.14) (end 59.86018 101.49332) (width 0.5) (layer F.Cu) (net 7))
 (segment (start 59.86018 101.49332) (end 60.0075 101.346) (width 0.5) (layer F.Cu) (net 7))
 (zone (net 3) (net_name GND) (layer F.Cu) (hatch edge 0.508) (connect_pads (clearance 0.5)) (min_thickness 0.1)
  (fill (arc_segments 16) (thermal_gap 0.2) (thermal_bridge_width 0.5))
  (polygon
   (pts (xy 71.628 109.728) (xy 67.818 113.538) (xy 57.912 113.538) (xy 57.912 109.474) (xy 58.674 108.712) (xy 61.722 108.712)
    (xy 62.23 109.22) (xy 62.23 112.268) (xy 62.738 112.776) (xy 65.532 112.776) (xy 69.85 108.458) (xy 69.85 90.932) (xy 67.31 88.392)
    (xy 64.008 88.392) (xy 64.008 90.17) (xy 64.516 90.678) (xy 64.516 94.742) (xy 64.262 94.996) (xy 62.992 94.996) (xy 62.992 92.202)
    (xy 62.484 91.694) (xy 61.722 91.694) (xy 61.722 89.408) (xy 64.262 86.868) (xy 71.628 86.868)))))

